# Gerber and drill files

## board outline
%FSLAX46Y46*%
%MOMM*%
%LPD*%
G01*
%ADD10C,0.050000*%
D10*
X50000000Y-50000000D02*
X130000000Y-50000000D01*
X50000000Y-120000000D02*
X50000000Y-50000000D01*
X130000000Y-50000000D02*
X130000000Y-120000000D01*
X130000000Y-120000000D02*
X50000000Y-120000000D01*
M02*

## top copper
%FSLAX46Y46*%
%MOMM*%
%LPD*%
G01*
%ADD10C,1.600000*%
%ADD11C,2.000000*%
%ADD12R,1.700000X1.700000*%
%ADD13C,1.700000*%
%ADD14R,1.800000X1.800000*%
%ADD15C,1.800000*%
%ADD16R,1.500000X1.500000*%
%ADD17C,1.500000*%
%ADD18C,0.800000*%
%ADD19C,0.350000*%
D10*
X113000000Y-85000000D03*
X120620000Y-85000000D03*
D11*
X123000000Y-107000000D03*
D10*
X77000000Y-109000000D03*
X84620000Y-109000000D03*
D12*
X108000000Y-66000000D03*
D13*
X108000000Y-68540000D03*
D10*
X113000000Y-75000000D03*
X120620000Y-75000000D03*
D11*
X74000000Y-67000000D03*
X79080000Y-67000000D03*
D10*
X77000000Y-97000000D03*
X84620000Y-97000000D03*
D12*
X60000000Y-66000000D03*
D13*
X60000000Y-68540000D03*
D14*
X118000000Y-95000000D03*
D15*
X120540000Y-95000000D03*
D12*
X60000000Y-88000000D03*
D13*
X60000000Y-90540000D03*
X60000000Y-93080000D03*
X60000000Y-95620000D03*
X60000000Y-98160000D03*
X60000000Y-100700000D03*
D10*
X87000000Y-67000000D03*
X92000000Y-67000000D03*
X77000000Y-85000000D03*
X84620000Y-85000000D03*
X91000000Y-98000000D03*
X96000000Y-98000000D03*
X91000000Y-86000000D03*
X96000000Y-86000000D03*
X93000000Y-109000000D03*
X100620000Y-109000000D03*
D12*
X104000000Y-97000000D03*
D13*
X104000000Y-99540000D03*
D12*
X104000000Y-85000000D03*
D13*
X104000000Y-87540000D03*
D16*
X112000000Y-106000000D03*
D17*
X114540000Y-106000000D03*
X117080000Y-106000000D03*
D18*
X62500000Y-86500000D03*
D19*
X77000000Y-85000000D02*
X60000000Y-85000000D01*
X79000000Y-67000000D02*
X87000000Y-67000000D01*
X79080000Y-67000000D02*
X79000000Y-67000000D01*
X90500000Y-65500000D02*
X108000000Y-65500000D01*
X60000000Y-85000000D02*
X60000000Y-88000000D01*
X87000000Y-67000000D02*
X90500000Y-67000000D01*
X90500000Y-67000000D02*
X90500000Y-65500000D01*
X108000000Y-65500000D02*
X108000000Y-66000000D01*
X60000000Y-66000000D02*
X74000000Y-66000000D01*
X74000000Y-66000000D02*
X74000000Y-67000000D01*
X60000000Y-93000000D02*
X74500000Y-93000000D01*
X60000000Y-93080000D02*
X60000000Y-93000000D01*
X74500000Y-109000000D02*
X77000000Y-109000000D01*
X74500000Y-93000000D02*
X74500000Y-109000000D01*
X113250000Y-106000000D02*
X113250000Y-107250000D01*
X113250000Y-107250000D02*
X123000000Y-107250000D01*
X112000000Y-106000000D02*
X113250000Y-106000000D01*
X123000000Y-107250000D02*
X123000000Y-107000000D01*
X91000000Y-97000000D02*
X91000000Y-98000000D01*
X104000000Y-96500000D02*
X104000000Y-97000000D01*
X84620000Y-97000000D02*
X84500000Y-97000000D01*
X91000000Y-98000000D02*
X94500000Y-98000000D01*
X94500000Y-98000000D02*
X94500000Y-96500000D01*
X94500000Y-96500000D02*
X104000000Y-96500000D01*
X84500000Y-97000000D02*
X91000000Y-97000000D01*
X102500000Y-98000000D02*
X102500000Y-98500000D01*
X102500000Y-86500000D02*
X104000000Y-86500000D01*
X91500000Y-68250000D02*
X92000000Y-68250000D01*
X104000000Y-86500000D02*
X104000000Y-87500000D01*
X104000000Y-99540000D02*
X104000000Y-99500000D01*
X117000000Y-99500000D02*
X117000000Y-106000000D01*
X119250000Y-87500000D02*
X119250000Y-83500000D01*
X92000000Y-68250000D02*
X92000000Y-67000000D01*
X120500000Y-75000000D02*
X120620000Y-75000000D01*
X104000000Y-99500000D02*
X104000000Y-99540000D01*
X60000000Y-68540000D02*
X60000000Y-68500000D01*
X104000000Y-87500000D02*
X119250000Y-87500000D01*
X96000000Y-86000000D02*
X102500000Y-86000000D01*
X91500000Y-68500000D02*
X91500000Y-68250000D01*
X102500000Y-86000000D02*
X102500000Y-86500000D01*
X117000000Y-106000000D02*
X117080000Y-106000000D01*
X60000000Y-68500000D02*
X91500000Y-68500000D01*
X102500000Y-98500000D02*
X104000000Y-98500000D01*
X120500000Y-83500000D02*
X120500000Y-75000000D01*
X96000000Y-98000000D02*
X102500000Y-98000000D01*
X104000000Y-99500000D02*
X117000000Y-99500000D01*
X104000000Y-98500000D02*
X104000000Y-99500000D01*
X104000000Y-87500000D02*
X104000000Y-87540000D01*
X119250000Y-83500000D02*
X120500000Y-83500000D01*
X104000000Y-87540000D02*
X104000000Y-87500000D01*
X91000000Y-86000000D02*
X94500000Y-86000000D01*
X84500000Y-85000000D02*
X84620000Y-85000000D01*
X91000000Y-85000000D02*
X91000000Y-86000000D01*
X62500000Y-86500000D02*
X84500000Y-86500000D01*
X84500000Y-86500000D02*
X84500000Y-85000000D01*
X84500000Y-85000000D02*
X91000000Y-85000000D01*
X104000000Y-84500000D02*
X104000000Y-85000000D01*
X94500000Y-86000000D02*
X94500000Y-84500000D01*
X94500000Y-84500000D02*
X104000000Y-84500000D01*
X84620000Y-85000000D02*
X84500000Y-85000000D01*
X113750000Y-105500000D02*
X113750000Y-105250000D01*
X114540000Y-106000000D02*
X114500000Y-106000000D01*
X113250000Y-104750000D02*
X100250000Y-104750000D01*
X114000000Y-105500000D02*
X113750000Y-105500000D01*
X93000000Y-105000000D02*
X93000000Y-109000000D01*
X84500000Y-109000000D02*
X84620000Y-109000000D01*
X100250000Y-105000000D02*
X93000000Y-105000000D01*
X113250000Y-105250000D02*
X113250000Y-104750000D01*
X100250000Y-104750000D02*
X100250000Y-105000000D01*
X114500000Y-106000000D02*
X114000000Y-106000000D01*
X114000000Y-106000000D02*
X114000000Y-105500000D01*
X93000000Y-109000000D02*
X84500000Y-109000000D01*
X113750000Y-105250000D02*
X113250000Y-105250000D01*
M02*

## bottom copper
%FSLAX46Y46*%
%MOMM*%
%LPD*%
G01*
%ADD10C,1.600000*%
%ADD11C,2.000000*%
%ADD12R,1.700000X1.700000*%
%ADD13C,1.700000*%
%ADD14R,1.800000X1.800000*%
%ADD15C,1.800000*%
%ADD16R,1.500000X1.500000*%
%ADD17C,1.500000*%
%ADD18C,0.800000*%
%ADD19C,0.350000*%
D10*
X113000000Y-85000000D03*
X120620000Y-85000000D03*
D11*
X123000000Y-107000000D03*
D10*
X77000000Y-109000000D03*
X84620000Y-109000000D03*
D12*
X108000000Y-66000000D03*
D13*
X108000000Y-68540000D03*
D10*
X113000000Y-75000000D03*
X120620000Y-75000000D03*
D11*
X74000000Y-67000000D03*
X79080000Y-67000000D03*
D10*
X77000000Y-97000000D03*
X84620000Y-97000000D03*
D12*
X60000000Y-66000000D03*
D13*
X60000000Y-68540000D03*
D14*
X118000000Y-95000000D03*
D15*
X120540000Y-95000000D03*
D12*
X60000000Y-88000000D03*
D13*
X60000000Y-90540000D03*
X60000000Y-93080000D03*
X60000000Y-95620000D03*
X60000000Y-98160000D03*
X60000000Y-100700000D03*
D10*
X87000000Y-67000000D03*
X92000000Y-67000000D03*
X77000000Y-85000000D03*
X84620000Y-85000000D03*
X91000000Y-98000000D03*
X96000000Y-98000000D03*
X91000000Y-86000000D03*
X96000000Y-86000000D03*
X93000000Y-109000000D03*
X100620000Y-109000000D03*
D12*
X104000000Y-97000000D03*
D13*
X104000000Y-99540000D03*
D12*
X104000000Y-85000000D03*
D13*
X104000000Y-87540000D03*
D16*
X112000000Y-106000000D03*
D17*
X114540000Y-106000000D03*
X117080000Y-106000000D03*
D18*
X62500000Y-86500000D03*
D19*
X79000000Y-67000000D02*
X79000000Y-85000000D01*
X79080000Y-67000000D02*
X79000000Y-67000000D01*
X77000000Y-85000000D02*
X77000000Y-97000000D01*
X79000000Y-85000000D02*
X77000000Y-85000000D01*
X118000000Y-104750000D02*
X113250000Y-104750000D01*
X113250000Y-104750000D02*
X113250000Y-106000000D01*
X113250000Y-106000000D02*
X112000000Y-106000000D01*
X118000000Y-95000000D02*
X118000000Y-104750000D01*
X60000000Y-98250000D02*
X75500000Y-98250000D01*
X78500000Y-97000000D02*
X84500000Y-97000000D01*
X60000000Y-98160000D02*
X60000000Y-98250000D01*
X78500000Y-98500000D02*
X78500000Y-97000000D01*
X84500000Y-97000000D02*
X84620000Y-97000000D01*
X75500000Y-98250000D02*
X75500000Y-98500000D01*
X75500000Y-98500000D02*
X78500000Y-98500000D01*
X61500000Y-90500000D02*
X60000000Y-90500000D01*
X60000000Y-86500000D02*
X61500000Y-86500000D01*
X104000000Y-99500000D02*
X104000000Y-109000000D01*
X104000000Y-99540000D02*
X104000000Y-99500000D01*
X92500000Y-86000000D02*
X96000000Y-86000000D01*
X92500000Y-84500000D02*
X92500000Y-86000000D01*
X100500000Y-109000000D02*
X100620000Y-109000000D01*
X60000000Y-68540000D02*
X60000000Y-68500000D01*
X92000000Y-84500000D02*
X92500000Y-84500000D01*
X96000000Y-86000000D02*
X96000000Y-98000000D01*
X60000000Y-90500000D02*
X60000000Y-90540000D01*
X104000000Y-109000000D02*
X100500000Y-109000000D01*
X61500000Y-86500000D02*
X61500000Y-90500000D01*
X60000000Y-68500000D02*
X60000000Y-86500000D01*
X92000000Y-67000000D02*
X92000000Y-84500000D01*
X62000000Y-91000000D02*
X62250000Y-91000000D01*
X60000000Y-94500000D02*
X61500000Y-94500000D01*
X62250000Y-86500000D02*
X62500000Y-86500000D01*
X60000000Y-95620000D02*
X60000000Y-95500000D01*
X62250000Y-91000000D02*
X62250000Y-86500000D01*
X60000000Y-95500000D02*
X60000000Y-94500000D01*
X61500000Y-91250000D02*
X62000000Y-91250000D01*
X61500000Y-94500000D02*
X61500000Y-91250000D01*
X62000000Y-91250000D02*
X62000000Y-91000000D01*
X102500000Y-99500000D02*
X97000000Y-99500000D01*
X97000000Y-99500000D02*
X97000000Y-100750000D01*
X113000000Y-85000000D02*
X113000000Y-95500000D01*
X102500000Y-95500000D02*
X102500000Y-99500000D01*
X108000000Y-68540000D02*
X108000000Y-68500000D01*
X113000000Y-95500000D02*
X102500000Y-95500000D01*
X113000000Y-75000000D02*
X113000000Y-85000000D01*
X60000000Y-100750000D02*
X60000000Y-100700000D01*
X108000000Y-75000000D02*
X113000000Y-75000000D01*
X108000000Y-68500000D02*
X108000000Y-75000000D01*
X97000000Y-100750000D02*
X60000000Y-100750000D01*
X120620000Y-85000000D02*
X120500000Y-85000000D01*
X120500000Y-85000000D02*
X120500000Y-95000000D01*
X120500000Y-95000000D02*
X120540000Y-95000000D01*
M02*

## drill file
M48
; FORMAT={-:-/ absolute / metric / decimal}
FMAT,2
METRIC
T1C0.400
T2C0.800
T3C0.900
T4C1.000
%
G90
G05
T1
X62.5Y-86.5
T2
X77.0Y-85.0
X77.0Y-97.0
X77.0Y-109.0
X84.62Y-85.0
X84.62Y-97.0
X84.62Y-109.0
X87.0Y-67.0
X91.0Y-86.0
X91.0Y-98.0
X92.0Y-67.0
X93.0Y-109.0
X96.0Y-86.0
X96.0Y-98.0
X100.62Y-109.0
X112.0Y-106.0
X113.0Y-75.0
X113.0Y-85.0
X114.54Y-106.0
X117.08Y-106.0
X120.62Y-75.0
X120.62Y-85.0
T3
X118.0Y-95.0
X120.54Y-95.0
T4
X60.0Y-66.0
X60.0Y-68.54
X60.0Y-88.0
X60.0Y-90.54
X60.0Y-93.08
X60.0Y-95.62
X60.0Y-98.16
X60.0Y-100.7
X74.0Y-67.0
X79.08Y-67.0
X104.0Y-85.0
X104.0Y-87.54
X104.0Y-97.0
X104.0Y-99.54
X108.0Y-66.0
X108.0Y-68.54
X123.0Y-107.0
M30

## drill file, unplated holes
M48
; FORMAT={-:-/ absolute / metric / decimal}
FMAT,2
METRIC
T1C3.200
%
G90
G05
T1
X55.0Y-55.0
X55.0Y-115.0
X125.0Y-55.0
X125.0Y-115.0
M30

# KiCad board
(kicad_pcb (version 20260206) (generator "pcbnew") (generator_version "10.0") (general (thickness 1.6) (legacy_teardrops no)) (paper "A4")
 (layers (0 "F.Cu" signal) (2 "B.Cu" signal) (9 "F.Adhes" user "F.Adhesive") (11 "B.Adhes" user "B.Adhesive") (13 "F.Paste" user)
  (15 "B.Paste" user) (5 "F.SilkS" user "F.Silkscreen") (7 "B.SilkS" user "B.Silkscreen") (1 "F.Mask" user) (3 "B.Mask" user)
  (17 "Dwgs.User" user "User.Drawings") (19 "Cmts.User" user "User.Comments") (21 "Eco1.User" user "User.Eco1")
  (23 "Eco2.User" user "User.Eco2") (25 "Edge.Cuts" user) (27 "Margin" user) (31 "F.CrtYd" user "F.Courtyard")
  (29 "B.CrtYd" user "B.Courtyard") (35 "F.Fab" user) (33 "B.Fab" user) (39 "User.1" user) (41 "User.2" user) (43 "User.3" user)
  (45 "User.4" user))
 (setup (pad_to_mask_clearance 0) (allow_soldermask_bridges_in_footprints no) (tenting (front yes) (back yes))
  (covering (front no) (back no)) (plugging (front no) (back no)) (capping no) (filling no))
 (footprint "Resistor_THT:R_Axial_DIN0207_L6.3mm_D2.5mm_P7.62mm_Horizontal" (layer "F.Cu") (at 113 85)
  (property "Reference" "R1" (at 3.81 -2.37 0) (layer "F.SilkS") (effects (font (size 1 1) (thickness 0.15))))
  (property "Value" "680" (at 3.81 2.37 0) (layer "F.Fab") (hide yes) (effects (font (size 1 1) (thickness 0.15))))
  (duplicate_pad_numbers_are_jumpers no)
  (pad "1" thru_hole circle (at 0 0) (size 1.6 1.6) (drill 0.8) (layers "*.Cu" "*.Mask") (remove_unused_layers no) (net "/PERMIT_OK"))
  (pad "2" thru_hole circle (at 7.62 0) (size 1.6 1.6) (drill 0.8) (layers "*.Cu" "*.Mask") (remove_unused_layers no) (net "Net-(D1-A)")))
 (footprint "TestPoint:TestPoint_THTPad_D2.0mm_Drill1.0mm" (layer "F.Cu") (at 123 107)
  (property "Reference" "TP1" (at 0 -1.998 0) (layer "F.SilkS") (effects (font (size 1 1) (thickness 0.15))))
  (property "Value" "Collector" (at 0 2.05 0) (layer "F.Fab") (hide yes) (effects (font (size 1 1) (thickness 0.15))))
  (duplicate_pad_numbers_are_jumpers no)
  (pad "1" thru_hole circle (at 0 0) (size 2 2) (drill 1) (layers "*.Cu" "*.Mask") (remove_unused_layers no) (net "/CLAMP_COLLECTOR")))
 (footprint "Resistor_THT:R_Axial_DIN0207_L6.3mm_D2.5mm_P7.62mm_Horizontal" (layer "F.Cu") (at 77 109)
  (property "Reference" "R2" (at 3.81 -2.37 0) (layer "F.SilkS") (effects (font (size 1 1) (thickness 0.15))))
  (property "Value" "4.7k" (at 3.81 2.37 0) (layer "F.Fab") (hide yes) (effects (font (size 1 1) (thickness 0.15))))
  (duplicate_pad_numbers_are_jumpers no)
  (pad "1" thru_hole circle (at 0 0) (size 1.6 1.6) (drill 0.8) (layers "*.Cu" "*.Mask") (remove_unused_layers no) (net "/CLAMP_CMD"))
  (pad "2" thru_hole circle (at 7.62 0) (size 1.6 1.6) (drill 0.8) (layers "*.Cu" "*.Mask") (remove_unused_layers no) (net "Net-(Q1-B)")))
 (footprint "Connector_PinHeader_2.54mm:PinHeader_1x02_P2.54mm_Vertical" (layer "F.Cu") (at 108 66)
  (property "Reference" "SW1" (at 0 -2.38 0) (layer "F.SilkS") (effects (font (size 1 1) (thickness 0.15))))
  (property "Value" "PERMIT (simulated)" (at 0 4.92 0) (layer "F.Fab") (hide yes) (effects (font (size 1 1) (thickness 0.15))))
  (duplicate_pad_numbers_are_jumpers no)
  (pad "1" thru_hole rect (at 0 0) (size 1.7 1.7) (drill 1) (layers "*.Cu" "*.Mask") (remove_unused_layers no) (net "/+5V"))
  (pad "2" thru_hole circle (at 0 2.54) (size 1.7 1.7) (drill 1) (layers "*.Cu" "*.Mask") (remove_unused_layers no) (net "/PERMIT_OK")))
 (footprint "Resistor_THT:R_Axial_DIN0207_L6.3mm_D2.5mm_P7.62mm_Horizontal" (layer "F.Cu") (at 113 75)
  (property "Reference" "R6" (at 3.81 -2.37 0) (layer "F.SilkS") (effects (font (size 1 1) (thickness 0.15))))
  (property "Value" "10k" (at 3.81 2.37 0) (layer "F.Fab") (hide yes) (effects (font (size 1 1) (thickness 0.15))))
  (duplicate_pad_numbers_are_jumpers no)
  (pad "1" thru_hole circle (at 0 0) (size 1.6 1.6) (drill 0.8) (layers "*.Cu" "*.Mask") (remove_unused_layers no) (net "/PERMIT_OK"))
  (pad "2" thru_hole circle (at 7.62 0) (size 1.6 1.6) (drill 0.8) (layers "*.Cu" "*.Mask") (remove_unused_layers no) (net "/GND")))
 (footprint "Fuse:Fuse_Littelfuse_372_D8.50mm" (layer "F.Cu") (at 74 67)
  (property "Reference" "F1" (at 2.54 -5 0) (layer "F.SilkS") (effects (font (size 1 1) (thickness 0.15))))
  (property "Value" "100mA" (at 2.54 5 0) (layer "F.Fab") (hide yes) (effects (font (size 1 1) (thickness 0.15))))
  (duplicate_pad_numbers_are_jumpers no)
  (pad "1" thru_hole circle (at 0 0) (size 2 2) (drill 1) (layers "*.Cu" "*.Mask") (remove_unused_layers no) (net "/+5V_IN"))
  (pad "2" thru_hole circle (at 5.08 0) (size 2 2) (drill 1) (layers "*.Cu" "*.Mask") (remove_unused_layers no) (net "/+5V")))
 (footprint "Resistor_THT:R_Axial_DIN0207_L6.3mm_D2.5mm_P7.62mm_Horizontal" (layer "F.Cu") (at 77 97)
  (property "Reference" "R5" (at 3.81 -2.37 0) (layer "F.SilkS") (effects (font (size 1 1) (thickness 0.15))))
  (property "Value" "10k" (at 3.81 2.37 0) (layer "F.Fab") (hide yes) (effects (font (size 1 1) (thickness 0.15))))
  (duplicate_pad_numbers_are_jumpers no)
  (pad "1" thru_hole circle (at 0 0) (size 1.6 1.6) (drill 0.8) (layers "*.Cu" "*.Mask") (remove_unused_layers no) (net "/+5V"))
  (pad "2" thru_hole circle (at 7.62 0) (size 1.6 1.6) (drill 0.8) (layers "*.Cu" "*.Mask") (remove_unused_layers no) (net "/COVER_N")))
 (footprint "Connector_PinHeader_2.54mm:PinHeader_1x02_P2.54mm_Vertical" (layer "F.Cu") (at 60 66)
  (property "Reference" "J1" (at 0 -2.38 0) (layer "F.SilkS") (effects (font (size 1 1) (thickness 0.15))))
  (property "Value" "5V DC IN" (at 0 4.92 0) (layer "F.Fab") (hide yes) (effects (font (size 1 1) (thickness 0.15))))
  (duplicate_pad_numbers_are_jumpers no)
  (pad "1" thru_hole rect (at 0 0) (size 1.7 1.7) (drill 1) (layers "*.Cu" "*.Mask") (remove_unused_layers no) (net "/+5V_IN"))
  (pad "2" thru_hole circle (at 0 2.54) (size 1.7 1.7) (drill 1) (layers "*.Cu" "*.Mask") (remove_unused_layers no) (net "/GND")))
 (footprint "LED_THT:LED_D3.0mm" (layer "F.Cu") (at 118 95)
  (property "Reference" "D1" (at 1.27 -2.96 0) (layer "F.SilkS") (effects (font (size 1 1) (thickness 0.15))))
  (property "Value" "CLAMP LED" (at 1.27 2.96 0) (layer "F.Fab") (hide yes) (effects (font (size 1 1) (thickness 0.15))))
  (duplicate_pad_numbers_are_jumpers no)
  (pad "1" thru_hole rect (at 0 0) (size 1.8 1.8) (drill 0.9) (layers "*.Cu" "*.Mask") (remove_unused_layers no) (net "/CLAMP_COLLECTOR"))
  (pad "2" thru_hole circle (at 2.54 0) (size 1.8 1.8) (drill 0.9) (layers "*.Cu" "*.Mask") (remove_unused_layers no) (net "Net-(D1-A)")))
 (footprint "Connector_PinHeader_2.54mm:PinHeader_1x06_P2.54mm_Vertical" (layer "F.Cu") (at 60 88)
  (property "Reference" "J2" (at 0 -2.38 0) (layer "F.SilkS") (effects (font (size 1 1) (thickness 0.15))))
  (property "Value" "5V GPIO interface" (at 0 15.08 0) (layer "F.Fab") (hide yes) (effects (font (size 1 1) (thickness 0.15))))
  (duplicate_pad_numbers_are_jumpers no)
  (pad "1" thru_hole rect (at 0 0) (size 1.7 1.7) (drill 1) (layers "*.Cu" "*.Mask") (remove_unused_layers no) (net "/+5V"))
  (pad "2" thru_hole circle (at 0 2.54) (size 1.7 1.7) (drill 1) (layers "*.Cu" "*.Mask") (remove_unused_layers no) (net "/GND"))
  (pad "3" thru_hole circle (at 0 5.08) (size 1.7 1.7) (drill 1) (layers "*.Cu" "*.Mask") (remove_unused_layers no) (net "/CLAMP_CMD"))
  (pad "4" thru_hole circle (at 0 7.62) (size 1.7 1.7) (drill 1) (layers "*.Cu" "*.Mask") (remove_unused_layers no) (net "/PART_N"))
  (pad "5" thru_hole circle (at 0 10.16) (size 1.7 1.7) (drill 1) (layers "*.Cu" "*.Mask") (remove_unused_layers no) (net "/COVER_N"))
  (pad "6" thru_hole circle (at 0 12.7) (size 1.7 1.7) (drill 1) (layers "*.Cu" "*.Mask") (remove_unused_layers no) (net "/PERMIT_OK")))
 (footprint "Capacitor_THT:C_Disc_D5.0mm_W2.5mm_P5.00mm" (layer "F.Cu") (at 87 67)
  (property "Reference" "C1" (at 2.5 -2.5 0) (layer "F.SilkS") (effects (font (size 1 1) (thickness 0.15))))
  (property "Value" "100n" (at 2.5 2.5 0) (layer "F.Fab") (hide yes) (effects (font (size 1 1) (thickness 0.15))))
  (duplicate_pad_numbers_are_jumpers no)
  (pad "1" thru_hole circle (at 0 0) (size 1.6 1.6) (drill 0.8) (layers "*.Cu" "*.Mask") (remove_unused_layers no) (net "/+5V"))
  (pad "2" thru_hole circle (at 5 0) (size 1.6 1.6) (drill 0.8) (layers "*.Cu" "*.Mask") (remove_unused_layers no) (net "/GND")))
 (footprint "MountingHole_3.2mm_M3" (layer "F.Cu") (at 55 115)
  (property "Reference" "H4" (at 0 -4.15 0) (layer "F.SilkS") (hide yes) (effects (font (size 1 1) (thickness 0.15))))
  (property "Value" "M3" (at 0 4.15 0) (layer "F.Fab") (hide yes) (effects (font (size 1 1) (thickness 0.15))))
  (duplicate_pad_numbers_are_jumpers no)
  (pad "" np_thru_hole circle (at 0 0) (size 3.2 3.2) (drill 3.2) (layers "*.Cu" "*.Mask")))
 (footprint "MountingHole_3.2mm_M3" (layer "F.Cu") (at 125 55)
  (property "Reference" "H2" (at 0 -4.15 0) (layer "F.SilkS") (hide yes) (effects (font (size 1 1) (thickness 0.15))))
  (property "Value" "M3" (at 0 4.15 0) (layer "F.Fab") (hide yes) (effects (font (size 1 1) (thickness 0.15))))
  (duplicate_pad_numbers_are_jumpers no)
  (pad "" np_thru_hole circle (at 0 0) (size 3.2 3.2) (drill 3.2) (layers "*.Cu" "*.Mask")))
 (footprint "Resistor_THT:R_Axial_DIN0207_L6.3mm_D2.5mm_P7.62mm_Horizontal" (layer "F.Cu") (at 77 85)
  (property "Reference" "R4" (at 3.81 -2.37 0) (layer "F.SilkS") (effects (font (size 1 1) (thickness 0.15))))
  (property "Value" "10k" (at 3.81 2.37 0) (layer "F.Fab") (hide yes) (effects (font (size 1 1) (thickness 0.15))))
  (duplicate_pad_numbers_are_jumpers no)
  (pad "1" thru_hole circle (at 0 0) (size 1.6 1.6) (drill 0.8) (layers "*.Cu" "*.Mask") (remove_unused_layers no) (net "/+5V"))
  (pad "2" thru_hole circle (at 7.62 0) (size 1.6 1.6) (drill 0.8) (layers "*.Cu" "*.Mask") (remove_unused_layers no) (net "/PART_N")))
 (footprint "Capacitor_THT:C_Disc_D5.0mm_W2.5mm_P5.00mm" (layer "F.Cu") (at 91 98)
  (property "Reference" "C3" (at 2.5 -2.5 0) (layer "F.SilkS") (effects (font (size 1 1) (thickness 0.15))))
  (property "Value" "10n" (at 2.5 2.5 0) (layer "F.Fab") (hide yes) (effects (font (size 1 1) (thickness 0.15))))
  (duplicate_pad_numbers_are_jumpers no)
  (pad "1" thru_hole circle (at 0 0) (size 1.6 1.6) (drill 0.8) (layers "*.Cu" "*.Mask") (remove_unused_layers no) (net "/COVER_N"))
  (pad "2" thru_hole circle (at 5 0) (size 1.6 1.6) (drill 0.8) (layers "*.Cu" "*.Mask") (remove_unused_layers no) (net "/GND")))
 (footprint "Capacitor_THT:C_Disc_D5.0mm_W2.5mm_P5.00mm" (layer "F.Cu") (at 91 86)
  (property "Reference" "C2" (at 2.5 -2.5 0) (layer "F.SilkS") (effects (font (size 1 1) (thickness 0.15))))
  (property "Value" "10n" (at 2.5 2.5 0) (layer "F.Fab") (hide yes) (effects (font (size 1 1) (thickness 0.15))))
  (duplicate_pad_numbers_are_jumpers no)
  (pad "1" thru_hole circle (at 0 0) (size 1.6 1.6) (drill 0.8) (layers "*.Cu" "*.Mask") (remove_unused_layers no) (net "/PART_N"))
  (pad "2" thru_hole circle (at 5 0) (size 1.6 1.6) (drill 0.8) (layers "*.Cu" "*.Mask") (remove_unused_layers no) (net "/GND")))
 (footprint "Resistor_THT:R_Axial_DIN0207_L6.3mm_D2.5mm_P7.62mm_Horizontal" (layer "F.Cu") (at 93 109)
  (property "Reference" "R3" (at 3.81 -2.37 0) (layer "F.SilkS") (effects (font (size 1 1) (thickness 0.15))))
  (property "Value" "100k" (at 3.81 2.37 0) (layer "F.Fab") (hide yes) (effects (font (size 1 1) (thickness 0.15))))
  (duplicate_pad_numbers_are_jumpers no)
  (pad "1" thru_hole circle (at 0 0) (size 1.6 1.6) (drill 0.8) (layers "*.Cu" "*.Mask") (remove_unused_layers no) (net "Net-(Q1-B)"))
  (pad "2" thru_hole circle (at 7.62 0) (size 1.6 1.6) (drill 0.8) (layers "*.Cu" "*.Mask") (remove_unused_layers no) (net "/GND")))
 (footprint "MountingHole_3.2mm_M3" (layer "F.Cu") (at 55 55)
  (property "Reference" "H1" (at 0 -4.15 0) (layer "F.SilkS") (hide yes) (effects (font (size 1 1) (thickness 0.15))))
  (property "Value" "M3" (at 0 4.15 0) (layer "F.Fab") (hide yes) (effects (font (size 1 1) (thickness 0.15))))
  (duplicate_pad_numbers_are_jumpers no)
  (pad "" np_thru_hole circle (at 0 0) (size 3.2 3.2) (drill 3.2) (layers "*.Cu" "*.Mask")))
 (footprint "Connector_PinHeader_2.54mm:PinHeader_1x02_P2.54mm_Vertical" (layer "F.Cu") (at 104 97)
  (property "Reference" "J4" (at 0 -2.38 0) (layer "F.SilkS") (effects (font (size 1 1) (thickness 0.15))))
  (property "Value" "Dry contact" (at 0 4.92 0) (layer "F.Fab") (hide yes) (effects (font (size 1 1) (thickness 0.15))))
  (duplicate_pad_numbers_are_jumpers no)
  (pad "1" thru_hole rect (at 0 0) (size 1.7 1.7) (drill 1) (layers "*.Cu" "*.Mask") (remove_unused_layers no) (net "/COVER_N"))
  (pad "2" thru_hole circle (at 0 2.54) (size 1.7 1.7) (drill 1) (layers "*.Cu" "*.Mask") (remove_unused_layers no) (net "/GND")))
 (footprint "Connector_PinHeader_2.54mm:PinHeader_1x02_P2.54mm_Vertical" (layer "F.Cu") (at 104 85)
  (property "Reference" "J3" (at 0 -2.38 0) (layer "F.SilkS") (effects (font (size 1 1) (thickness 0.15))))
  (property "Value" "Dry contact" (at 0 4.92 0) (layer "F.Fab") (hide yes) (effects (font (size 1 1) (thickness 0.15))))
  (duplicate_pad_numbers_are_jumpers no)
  (pad "1" thru_hole rect (at 0 0) (size 1.7 1.7) (drill 1) (layers "*.Cu" "*.Mask") (remove_unused_layers no) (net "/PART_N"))
  (pad "2" thru_hole circle (at 0 2.54) (size 1.7 1.7) (drill 1) (layers "*.Cu" "*.Mask") (remove_unused_layers no) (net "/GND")))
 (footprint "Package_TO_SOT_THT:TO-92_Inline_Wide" (layer "F.Cu") (at 112 106)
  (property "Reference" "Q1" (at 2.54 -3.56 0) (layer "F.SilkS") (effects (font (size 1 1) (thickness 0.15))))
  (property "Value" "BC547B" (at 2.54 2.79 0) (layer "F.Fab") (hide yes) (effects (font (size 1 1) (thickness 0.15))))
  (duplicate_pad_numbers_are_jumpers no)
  (pad "1" thru_hole rect (at 0 0) (size 1.5 1.5) (drill 0.8) (layers "*.Cu" "*.Mask") (remove_unused_layers no) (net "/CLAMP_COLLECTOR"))
  (pad "2" thru_hole circle (at 2.54 0) (size 1.5 1.5) (drill 0.8) (layers "*.Cu" "*.Mask") (remove_unused_layers no) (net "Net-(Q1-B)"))
  (pad "3" thru_hole circle (at 5.08 0) (size 1.5 1.5) (drill 0.8) (layers "*.Cu" "*.Mask") (remove_unused_layers no) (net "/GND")))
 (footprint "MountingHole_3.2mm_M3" (layer "F.Cu") (at 125 115)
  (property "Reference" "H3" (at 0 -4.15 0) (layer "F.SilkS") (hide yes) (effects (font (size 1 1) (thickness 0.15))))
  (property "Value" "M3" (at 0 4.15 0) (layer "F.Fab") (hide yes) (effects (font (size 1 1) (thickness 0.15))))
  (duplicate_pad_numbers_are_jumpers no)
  (pad "" np_thru_hole circle (at 0 0) (size 3.2 3.2) (drill 3.2) (layers "*.Cu" "*.Mask")))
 (gr_line (start 50 50) (end 130 50) (stroke (width 0.05) (type default)) (layer "Edge.Cuts"))
 (gr_line (start 50 120) (end 50 50) (stroke (width 0.05) (type default)) (layer "Edge.Cuts"))
 (gr_line (start 130 50) (end 130 120) (stroke (width 0.05) (type default)) (layer "Edge.Cuts"))
 (gr_line (start 130 120) (end 50 120) (stroke (width 0.05) (type default)) (layer "Edge.Cuts"))
 (segment (start 77 85) (end 60 85) (width 0.35) (layer "F.Cu") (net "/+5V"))
 (segment (start 79 67) (end 87 67) (width 0.35) (layer "F.Cu") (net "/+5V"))
 (segment (start 79.08 67) (end 79 67) (width 0.35) (layer "F.Cu") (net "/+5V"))
 (segment (start 90.5 65.5) (end 108 65.5) (width 0.35) (layer "F.Cu") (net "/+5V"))
 (segment (start 60 85) (end 60 88) (width 0.35) (layer "F.Cu") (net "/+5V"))
 (segment (start 87 67) (end 90.5 67) (width 0.35) (layer "F.Cu") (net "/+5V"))
 (segment (start 90.5 67) (end 90.5 65.5) (width 0.35) (layer "F.Cu") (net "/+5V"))
 (segment (start 108 65.5) (end 108 66) (width 0.35) (layer "F.Cu") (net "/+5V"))
 (segment (start 79 67) (end 79 85) (width 0.35) (layer "B.Cu") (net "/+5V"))
 (segment (start 79.08 67) (end 79 67) (width 0.35) (layer "B.Cu") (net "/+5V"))
 (segment (start 77 85) (end 77 97) (width 0.35) (layer "B.Cu") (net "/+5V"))
 (segment (start 79 85) (end 77 85) (width 0.35) (layer "B.Cu") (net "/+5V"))
 (segment (start 60 66) (end 74 66) (width 0.35) (layer "F.Cu") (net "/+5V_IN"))
 (segment (start 74 66) (end 74 67) (width 0.35) (layer "F.Cu") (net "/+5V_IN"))
 (segment (start 60 93) (end 74.5 93) (width 0.35) (layer "F.Cu") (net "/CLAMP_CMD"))
 (segment (start 60 93.08) (end 60 93) (width 0.35) (layer "F.Cu") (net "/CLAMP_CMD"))
 (segment (start 74.5 109) (end 77 109) (width 0.35) (layer "F.Cu") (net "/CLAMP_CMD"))
 (segment (start 74.5 93) (end 74.5 109) (width 0.35) (layer "F.Cu") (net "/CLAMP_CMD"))
 (segment (start 113.25 106) (end 113.25 107.25) (width 0.35) (layer "F.Cu") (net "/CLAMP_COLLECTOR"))
 (segment (start 113.25 107.25) (end 123 107.25) (width 0.35) (layer "F.Cu") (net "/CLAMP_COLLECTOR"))
 (segment (start 112 106) (end 113.25 106) (width 0.35) (layer "F.Cu") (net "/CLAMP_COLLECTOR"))
 (segment (start 123 107.25) (end 123 107) (width 0.35) (layer "F.Cu") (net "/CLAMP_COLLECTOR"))
 (segment (start 118 104.75) (end 113.25 104.75) (width 0.35) (layer "B.Cu") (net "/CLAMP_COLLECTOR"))
 (segment (start 113.25 104.75) (end 113.25 106) (width 0.35) (layer "B.Cu") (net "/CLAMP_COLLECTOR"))
 (segment (start 113.25 106) (end 112 106) (width 0.35) (layer "B.Cu") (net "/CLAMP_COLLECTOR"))
 (segment (start 118 95) (end 118 104.75) (width 0.35) (layer "B.Cu") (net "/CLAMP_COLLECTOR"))
 (segment (start 91 97) (end 91 98) (width 0.35) (layer "F.Cu") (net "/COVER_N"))
 (segment (start 104 96.5) (end 104 97) (width 0.35) (layer "F.Cu") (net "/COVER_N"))
 (segment (start 84.62 97) (end 84.5 97) (width 0.35) (layer "F.Cu") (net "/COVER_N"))
 (segment (start 91 98) (end 94.5 98) (width 0.35) (layer "F.Cu") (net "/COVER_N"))
 (segment (start 94.5 98) (end 94.5 96.5) (width 0.35) (layer "F.Cu") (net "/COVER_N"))
 (segment (start 94.5 96.5) (end 104 96.5) (width 0.35) (layer "F.Cu") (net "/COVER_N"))
 (segment (start 84.5 97) (end 91 97) (width 0.35) (layer "F.Cu") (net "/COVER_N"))
 (segment (start 60 98.25) (end 75.5 98.25) (width 0.35) (layer "B.Cu") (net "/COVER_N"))
 (segment (start 78.5 97) (end 84.5 97) (width 0.35) (layer "B.Cu") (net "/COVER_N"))
 (segment (start 60 98.16) (end 60 98.25) (width 0.35) (layer "B.Cu") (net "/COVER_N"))
 (segment (start 78.5 98.5) (end 78.5 97) (width 0.35) (layer "B.Cu") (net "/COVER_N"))
 (segment (start 84.5 97) (end 84.62 97) (width 0.35) (layer "B.Cu") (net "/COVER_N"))
 (segment (start 75.5 98.25) (end 75.5 98.5) (width 0.35) (layer "B.Cu") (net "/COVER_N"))
 (segment (start 75.5 98.5) (end 78.5 98.5) (width 0.35) (layer "B.Cu") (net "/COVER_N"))
 (segment (start 102.5 98) (end 102.5 98.5) (width 0.35) (layer "F.Cu") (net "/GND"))
 (segment (start 102.5 86.5) (end 104 86.5) (width 0.35) (layer "F.Cu") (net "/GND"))
 (segment (start 91.5 68.25) (end 92 68.25) (width 0.35) (layer "F.Cu") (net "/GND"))
 (segment (start 104 86.5) (end 104 87.5) (width 0.35) (layer "F.Cu") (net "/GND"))
 (segment (start 104 99.54) (end 104 99.5) (width 0.35) (layer "F.Cu") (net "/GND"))
 (segment (start 117 99.5) (end 117 106) (width 0.35) (layer "F.Cu") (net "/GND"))
 (segment (start 119.25 87.5) (end 119.25 83.5) (width 0.35) (layer "F.Cu") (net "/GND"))
 (segment (start 92 68.25) (end 92 67) (width 0.35) (layer "F.Cu") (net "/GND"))
 (segment (start 120.5 75) (end 120.62 75) (width 0.35) (layer "F.Cu") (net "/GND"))
 (segment (start 104 99.5) (end 104 99.54) (width 0.35) (layer "F.Cu") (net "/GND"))
 (segment (start 60 68.54) (end 60 68.5) (width 0.35) (layer "F.Cu") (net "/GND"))
 (segment (start 104 87.5) (end 119.25 87.5) (width 0.35) (layer "F.Cu") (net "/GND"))
 (segment (start 96 86) (end 102.5 86) (width 0.35) (layer "F.Cu") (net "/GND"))
 (segment (start 91.5 68.5) (end 91.5 68.25) (width 0.35) (layer "F.Cu") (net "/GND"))
 (segment (start 102.5 86) (end 102.5 86.5) (width 0.35) (layer "F.Cu") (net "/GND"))
 (segment (start 117 106) (end 117.08 106) (width 0.35) (layer "F.Cu") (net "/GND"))
 (segment (start 60 68.5) (end 91.5 68.5) (width 0.35) (layer "F.Cu") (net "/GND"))
 (segment (start 102.5 98.5) (end 104 98.5) (width 0.35) (layer "F.Cu") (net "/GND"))
 (segment (start 120.5 83.5) (end 120.5 75) (width 0.35) (layer "F.Cu") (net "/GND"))
 (segment (start 96 98) (end 102.5 98) (width 0.35) (layer "F.Cu") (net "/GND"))
 (segment (start 104 99.5) (end 117 99.5) (width 0.35) (layer "F.Cu") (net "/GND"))
 (segment (start 104 98.5) (end 104 99.5) (width 0.35) (layer "F.Cu") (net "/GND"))
 (segment (start 104 87.5) (end 104 87.54) (width 0.35) (layer "F.Cu") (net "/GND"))
 (segment (start 119.25 83.5) (end 120.5 83.5) (width 0.35) (layer "F.Cu") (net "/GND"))
 (segment (start 104 87.54) (end 104 87.5) (width 0.35) (layer "F.Cu") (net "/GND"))
 (segment (start 61.5 90.5) (end 60 90.5) (width 0.35) (layer "B.Cu") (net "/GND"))
 (segment (start 60 86.5) (end 61.5 86.5) (width 0.35) (layer "B.Cu") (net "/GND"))
 (segment (start 104 99.5) (end 104 109) (width 0.35) (layer "B.Cu") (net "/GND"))
 (segment (start 104 99.54) (end 104 99.5) (width 0.35) (layer "B.Cu") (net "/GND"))
 (segment (start 92.5 86) (end 96 86) (width 0.35) (layer "B.Cu") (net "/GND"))
 (segment (start 92.5 84.5) (end 92.5 86) (width 0.35) (layer "B.Cu") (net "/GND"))
 (segment (start 100.5 109) (end 100.62 109) (width 0.35) (layer "B.Cu") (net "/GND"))
 (segment (start 60 68.54) (end 60 68.5) (width 0.35) (layer "B.Cu") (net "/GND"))
 (segment (start 92 84.5) (end 92.5 84.5) (width 0.35) (layer "B.Cu") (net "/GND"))
 (segment (start 96 86) (end 96 98) (width 0.35) (layer "B.Cu") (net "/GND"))
 (segment (start 60 90.5) (end 60 90.54) (width 0.35) (layer "B.Cu") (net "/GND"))
 (segment (start 104 109) (end 100.5 109) (width 0.35) (layer "B.Cu") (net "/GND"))
 (segment (start 61.5 86.5) (end 61.5 90.5) (width 0.35) (layer "B.Cu") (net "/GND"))
 (segment (start 60 68.5) (end 60 86.5) (width 0.35) (layer "B.Cu") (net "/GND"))
 (segment (start 92 67) (end 92 84.5) (width 0.35) (layer "B.Cu") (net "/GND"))
 (segment (start 91 86) (end 94.5 86) (width 0.35) (layer "F.Cu") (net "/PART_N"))
 (segment (start 84.5 85) (end 84.62 85) (width 0.35) (layer "F.Cu") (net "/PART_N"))
 (segment (start 91 85) (end 91 86) (width 0.35) (layer "F.Cu") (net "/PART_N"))
 (segment (start 62.5 86.5) (end 84.5 86.5) (width 0.35) (layer "F.Cu") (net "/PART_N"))
 (segment (start 84.5 86.5) (end 84.5 85) (width 0.35) (layer "F.Cu") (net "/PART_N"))
 (segment (start 84.5 85) (end 91 85) (width 0.35) (layer "F.Cu") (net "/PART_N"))
 (segment (start 104 84.5) (end 104 85) (width 0.35) (layer "F.Cu") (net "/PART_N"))
 (segment (start 94.5 86) (end 94.5 84.5) (width 0.35) (layer "F.Cu") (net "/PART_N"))
 (segment (start 94.5 84.5) (end 104 84.5) (width 0.35) (layer "F.Cu") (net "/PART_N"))
 (segment (start 84.62 85) (end 84.5 85) (width 0.35) (layer "F.Cu") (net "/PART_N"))
 (via (at 62.5 86.5) (size 0.8) (drill 0.4) (layers "F.Cu" "B.Cu") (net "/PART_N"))
 (segment (start 62 91) (end 62.25 91) (width 0.35) (layer "B.Cu") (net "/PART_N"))
 (segment (start 60 94.5) (end 61.5 94.5) (width 0.35) (layer "B.Cu") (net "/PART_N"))
 (segment (start 62.25 86.5) (end 62.5 86.5) (width 0.35) (layer "B.Cu") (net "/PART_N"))
 (segment (start 60 95.62) (end 60 95.5) (width 0.35) (layer "B.Cu") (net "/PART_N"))
 (segment (start 62.25 91) (end 62.25 86.5) (width 0.35) (layer "B.Cu") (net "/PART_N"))
 (segment (start 60 95.5) (end 60 94.5) (width 0.35) (layer "B.Cu") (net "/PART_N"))
 (segment (start 61.5 91.25) (end 62 91.25) (width 0.35) (layer "B.Cu") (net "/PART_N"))
 (segment (start 61.5 94.5) (end 61.5 91.25) (width 0.35) (layer "B.Cu") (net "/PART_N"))
 (segment (start 62 91.25) (end 62 91) (width 0.35) (layer "B.Cu") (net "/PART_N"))
 (segment (start 102.5 99.5) (end 97 99.5) (width 0.35) (layer "B.Cu") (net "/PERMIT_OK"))
 (segment (start 97 99.5) (end 97 100.75) (width 0.35) (layer "B.Cu") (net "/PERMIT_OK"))
 (segment (start 113 85) (end 113 95.5) (width 0.35) (layer "B.Cu") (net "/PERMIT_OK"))
 (segment (start 102.5 95.5) (end 102.5 99.5) (width 0.35) (layer "B.Cu") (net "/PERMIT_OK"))
 (segment (start 108 68.54) (end 108 68.5) (width 0.35) (layer "B.Cu") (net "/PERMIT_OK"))
 (segment (start 113 95.5) (end 102.5 95.5) (width 0.35) (layer "B.Cu") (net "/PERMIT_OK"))
 (segment (start 113 75) (end 113 85) (width 0.35) (layer "B.Cu") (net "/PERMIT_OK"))
 (segment (start 60 100.75) (end 60 100.7) (width 0.35) (layer "B.Cu") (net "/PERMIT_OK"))
 (segment (start 108 75) (end 113 75) (width 0.35) (layer "B.Cu") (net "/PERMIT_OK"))
 (segment (start 108 68.5) (end 108 75) (width 0.35) (layer "B.Cu") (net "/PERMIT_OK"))
 (segment (start 97 100.75) (end 60 100.75) (width 0.35) (layer "B.Cu") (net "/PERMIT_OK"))
 (segment (start 120.62 85) (end 120.5 85) (width 0.35) (layer "B.Cu") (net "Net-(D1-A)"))
 (segment (start 120.5 85) (end 120.5 95) (width 0.35) (layer "B.Cu") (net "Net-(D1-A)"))
 (segment (start 120.5 95) (end 120.54 95) (width 0.35) (layer "B.Cu") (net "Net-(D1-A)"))
 (segment (start 113.75 105.5) (end 113.75 105.25) (width 0.35) (layer "F.Cu") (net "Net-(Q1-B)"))
 (segment (start 114.54 106) (end 114.5 106) (width 0.35) (layer "F.Cu") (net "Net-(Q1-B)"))
 (segment (start 113.25 104.75) (end 100.25 104.75) (width 0.35) (layer "F.Cu") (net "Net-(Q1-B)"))
 (segment (start 114 105.5) (end 113.75 105.5) (width 0.35) (layer "F.Cu") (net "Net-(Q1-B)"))
 (segment (start 93 105) (end 93 109) (width 0.35) (layer "F.Cu") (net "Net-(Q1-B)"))
 (segment (start 84.5 109) (end 84.62 109) (width 0.35) (layer "F.Cu") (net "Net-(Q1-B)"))
 (segment (start 100.25 105) (end 93 105) (width 0.35) (layer "F.Cu") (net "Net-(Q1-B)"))
 (segment (start 113.25 105.25) (end 113.25 104.75) (width 0.35) (layer "F.Cu") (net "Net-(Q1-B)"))
 (segment (start 100.25 104.75) (end 100.25 105) (width 0.35) (layer "F.Cu") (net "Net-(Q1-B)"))
 (segment (start 114.5 106) (end 114 106) (width 0.35) (layer "F.Cu") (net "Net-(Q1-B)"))
 (segment (start 114 106) (end 114 105.5) (width 0.35) (layer "F.Cu") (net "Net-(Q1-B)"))
 (segment (start 93 109) (end 84.5 109) (width 0.35) (layer "F.Cu") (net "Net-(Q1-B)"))
 (segment (start 113.75 105.25) (end 113.25 105.25) (width 0.35) (layer "F.Cu") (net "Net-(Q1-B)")))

